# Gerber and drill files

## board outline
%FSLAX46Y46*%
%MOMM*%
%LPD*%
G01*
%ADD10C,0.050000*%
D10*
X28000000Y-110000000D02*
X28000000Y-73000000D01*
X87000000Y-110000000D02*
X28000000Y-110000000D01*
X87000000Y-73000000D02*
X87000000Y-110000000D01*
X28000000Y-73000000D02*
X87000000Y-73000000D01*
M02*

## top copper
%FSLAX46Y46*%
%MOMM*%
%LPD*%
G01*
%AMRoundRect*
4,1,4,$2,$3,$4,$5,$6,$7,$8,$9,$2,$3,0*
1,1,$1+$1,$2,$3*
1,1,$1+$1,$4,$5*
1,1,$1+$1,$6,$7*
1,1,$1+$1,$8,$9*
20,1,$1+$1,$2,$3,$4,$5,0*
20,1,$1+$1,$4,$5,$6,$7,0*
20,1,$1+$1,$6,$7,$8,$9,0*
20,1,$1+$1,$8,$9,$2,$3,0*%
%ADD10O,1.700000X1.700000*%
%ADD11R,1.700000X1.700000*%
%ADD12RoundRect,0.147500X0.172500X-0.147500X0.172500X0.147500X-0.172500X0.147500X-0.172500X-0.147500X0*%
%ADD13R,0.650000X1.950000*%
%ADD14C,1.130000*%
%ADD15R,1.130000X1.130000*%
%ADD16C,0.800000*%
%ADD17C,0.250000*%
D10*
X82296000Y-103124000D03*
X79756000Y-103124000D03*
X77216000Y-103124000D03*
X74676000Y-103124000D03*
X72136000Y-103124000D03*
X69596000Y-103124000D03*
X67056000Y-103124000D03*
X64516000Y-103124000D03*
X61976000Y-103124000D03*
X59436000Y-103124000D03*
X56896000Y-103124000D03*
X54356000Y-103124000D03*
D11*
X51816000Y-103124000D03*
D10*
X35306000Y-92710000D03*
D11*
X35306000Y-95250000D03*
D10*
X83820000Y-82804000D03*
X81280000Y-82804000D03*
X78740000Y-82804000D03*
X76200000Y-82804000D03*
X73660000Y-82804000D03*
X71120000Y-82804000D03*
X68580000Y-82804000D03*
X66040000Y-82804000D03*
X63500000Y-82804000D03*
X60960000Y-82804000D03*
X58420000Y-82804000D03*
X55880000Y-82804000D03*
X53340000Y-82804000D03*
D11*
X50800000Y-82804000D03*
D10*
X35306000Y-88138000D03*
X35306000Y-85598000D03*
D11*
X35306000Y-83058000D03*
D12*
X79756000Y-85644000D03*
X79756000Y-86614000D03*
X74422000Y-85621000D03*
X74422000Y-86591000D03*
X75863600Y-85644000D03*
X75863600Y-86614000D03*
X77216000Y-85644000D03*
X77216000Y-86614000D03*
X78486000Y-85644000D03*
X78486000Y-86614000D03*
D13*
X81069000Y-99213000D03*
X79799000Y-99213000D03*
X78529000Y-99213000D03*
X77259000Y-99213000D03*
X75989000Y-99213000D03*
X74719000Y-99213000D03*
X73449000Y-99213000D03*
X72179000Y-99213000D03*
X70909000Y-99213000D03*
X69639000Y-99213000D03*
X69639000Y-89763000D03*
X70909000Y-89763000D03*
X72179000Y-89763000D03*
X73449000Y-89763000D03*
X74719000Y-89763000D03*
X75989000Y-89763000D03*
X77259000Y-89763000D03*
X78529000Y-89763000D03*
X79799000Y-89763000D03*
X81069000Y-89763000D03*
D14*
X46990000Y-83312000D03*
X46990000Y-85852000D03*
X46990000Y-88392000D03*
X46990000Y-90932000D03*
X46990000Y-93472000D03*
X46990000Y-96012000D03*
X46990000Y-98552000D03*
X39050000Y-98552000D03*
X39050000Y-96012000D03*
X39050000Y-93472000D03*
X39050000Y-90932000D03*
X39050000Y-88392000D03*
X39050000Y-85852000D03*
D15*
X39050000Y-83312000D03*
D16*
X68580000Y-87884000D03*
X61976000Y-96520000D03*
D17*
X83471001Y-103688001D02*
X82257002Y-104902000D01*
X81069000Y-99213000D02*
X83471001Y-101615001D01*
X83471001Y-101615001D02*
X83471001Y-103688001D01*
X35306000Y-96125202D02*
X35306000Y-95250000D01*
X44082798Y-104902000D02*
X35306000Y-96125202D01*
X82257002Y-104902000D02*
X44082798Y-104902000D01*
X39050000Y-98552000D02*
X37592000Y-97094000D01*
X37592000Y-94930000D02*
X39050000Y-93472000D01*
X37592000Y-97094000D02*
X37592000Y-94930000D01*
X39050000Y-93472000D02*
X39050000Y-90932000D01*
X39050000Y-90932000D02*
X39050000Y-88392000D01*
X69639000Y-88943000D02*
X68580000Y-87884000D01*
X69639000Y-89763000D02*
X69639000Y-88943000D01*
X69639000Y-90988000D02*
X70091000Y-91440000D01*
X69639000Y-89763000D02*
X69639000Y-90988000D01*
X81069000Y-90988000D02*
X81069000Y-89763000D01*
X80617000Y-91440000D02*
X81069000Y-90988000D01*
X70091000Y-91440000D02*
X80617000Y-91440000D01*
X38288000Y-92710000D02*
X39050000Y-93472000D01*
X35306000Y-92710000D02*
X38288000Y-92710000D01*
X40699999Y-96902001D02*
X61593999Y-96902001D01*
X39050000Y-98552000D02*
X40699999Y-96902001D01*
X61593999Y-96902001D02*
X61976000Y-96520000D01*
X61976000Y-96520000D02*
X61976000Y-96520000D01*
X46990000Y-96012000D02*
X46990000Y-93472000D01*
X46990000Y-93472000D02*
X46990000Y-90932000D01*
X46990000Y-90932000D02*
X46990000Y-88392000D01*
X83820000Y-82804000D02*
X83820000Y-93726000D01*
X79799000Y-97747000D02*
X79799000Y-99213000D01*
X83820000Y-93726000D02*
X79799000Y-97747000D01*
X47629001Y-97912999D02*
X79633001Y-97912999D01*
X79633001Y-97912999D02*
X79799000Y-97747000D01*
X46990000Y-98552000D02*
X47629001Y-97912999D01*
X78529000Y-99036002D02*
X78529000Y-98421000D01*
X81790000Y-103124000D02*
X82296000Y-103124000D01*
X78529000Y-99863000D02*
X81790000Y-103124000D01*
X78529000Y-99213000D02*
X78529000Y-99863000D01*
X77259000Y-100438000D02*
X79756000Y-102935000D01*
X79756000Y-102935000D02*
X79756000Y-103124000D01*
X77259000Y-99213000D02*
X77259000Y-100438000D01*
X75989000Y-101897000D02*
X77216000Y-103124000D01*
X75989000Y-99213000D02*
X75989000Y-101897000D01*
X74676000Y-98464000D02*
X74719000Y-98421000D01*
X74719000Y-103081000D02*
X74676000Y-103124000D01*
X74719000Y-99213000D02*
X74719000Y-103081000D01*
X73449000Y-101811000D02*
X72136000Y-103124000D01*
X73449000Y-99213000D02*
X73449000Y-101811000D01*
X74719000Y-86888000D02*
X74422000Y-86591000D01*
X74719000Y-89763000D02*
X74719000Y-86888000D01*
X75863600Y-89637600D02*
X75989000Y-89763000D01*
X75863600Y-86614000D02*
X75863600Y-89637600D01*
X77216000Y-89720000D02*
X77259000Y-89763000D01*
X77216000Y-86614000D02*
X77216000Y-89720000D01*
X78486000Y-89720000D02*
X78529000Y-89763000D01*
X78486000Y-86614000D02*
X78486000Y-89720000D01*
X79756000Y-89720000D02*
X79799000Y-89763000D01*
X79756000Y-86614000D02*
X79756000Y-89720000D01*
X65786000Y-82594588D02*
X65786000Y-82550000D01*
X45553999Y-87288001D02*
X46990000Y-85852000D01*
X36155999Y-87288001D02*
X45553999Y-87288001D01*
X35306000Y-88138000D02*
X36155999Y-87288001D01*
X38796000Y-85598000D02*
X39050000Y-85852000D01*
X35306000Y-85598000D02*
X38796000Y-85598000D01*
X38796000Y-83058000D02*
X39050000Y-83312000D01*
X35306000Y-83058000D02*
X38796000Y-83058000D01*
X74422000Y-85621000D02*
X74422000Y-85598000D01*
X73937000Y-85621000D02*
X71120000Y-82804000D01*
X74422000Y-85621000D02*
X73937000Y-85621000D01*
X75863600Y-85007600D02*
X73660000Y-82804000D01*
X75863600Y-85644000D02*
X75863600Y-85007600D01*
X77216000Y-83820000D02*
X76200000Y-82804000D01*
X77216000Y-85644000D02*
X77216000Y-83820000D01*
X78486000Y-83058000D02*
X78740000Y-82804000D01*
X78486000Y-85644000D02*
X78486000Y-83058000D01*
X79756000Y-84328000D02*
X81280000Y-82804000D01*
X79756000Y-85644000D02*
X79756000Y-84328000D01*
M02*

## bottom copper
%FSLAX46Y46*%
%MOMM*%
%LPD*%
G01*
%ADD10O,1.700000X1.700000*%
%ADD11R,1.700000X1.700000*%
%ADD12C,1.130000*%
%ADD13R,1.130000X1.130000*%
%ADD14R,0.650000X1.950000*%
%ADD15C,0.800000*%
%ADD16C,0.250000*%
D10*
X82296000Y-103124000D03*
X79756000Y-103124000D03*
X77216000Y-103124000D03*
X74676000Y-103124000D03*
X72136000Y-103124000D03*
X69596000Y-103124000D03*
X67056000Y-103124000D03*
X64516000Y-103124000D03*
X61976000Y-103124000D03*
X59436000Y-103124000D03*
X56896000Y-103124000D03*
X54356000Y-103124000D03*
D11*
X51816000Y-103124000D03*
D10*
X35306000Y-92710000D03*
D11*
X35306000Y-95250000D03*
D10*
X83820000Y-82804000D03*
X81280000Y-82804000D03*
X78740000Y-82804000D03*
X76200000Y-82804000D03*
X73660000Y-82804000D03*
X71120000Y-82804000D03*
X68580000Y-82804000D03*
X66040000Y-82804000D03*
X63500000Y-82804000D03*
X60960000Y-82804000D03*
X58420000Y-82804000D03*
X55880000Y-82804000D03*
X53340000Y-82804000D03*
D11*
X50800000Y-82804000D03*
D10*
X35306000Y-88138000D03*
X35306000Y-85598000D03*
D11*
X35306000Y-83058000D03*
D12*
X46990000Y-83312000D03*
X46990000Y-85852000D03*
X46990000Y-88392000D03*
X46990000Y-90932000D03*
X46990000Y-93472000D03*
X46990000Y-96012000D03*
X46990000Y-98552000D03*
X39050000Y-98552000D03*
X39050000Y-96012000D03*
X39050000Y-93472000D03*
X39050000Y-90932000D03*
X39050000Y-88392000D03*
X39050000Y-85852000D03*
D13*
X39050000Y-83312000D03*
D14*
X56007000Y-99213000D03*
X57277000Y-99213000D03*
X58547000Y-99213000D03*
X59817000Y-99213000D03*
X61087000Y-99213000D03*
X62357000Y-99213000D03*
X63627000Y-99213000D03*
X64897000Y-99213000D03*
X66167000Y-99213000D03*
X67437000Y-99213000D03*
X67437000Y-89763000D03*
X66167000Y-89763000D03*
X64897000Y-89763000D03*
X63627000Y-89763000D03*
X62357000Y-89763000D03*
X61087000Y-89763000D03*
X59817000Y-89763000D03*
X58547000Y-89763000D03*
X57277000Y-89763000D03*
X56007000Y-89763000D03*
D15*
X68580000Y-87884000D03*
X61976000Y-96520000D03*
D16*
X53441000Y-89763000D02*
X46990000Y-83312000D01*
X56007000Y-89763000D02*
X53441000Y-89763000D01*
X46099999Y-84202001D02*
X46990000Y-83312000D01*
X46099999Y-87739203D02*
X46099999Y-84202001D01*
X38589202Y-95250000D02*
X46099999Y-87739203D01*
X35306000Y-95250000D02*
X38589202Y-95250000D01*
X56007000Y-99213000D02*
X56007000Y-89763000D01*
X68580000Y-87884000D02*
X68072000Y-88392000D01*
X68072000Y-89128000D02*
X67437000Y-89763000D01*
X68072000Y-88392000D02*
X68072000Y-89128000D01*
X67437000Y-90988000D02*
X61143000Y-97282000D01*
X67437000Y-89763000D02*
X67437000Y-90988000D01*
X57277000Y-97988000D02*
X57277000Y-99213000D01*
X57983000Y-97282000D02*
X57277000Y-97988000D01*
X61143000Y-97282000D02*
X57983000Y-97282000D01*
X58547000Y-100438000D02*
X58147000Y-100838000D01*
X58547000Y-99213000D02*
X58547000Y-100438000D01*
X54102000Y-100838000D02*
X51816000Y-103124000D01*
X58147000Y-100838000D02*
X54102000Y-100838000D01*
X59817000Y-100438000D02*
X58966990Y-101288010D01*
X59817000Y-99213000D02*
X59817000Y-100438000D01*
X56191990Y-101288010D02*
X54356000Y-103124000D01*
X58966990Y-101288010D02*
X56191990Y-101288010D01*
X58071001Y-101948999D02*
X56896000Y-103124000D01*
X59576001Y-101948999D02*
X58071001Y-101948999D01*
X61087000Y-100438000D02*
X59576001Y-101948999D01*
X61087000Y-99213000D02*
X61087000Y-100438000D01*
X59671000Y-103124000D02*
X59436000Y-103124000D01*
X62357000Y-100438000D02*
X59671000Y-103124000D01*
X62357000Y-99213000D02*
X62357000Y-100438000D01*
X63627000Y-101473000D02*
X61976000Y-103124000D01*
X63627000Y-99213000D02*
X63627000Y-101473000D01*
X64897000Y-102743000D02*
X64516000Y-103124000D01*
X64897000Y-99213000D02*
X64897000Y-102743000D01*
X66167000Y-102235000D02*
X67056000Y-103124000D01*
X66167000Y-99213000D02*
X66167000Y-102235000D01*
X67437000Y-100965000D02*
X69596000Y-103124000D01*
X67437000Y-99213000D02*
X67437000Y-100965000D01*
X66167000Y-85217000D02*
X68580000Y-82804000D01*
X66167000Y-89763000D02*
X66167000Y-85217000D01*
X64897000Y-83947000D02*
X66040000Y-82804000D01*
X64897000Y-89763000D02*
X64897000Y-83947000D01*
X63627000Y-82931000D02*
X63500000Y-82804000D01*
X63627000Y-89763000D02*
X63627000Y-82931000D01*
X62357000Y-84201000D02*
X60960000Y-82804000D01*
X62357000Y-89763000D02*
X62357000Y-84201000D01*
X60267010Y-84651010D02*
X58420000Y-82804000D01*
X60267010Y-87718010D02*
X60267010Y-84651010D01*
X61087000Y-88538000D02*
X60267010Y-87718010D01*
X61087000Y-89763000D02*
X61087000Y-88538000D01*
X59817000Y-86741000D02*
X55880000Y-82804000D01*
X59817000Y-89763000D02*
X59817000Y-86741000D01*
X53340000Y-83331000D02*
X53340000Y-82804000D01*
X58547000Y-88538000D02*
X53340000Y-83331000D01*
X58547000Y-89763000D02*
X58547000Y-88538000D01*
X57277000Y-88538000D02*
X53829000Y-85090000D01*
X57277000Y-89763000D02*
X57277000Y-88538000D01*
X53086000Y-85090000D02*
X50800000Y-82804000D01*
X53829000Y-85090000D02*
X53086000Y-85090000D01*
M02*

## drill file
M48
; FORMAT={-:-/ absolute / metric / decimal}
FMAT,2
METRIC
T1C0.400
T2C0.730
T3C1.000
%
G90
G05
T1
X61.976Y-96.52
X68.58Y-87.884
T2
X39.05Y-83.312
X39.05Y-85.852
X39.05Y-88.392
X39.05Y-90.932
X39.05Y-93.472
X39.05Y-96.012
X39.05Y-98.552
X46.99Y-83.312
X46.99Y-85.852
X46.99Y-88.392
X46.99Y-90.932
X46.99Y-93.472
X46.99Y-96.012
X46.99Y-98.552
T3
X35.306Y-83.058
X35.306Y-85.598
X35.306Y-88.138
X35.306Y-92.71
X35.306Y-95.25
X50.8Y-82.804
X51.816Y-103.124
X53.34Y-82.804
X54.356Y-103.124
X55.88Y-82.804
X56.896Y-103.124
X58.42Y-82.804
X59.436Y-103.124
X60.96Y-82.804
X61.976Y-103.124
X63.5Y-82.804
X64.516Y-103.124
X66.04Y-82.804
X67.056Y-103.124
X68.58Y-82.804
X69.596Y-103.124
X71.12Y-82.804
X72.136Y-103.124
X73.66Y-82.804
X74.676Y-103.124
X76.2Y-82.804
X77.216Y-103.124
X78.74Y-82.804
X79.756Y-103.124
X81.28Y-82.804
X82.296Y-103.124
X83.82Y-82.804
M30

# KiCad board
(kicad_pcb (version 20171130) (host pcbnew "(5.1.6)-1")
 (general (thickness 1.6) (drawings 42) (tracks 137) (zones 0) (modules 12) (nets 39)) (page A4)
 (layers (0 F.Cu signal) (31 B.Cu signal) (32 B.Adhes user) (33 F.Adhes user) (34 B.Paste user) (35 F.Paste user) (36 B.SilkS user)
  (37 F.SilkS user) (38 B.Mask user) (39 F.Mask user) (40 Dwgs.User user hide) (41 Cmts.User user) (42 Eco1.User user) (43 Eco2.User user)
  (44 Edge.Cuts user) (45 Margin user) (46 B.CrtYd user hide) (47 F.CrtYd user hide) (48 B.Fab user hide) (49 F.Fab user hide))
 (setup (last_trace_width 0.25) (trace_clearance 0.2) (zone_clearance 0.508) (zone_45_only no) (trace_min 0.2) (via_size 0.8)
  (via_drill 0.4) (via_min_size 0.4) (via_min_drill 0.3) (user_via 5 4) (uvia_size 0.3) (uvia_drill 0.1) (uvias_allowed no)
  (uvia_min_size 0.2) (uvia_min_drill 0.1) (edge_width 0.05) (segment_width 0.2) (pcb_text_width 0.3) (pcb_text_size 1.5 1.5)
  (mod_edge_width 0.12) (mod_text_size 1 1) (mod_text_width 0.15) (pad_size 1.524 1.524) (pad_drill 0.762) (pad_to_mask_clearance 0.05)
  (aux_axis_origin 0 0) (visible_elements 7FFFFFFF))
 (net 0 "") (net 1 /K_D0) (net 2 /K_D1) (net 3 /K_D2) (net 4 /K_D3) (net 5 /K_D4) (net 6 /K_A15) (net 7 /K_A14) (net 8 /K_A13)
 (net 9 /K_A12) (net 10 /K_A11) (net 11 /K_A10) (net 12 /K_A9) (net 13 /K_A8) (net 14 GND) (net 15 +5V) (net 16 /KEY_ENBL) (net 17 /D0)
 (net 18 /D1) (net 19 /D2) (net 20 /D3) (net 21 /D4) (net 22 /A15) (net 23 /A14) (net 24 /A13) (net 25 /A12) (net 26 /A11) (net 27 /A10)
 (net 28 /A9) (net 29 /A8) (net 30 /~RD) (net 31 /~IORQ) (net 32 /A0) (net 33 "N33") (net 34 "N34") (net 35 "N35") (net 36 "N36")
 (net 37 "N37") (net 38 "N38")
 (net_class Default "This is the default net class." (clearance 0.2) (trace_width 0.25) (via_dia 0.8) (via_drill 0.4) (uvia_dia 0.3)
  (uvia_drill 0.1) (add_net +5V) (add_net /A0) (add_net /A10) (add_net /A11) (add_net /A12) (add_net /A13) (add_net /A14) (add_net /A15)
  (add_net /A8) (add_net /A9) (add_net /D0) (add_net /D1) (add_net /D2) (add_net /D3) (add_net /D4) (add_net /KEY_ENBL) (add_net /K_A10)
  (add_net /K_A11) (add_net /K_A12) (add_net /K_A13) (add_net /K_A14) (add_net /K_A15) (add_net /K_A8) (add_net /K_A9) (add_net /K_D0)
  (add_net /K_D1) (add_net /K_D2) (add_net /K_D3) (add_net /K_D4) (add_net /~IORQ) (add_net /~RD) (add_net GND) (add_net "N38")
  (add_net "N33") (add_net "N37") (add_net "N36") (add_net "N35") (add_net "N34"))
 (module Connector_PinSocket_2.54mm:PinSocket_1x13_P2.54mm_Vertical (layer B.Cu) (at 51.816 103.124 270)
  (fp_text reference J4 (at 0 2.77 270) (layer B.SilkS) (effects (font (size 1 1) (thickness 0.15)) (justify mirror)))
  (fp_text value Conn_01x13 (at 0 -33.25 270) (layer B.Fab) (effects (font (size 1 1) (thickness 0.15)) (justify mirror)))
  (pad 13 thru_hole oval (at 0 -30.48 270) (size 1.7 1.7) (drill 1) (layers *.Cu *.Mask) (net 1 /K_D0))
  (pad 12 thru_hole oval (at 0 -27.94 270) (size 1.7 1.7) (drill 1) (layers *.Cu *.Mask) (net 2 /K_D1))
  (pad 11 thru_hole oval (at 0 -25.4 270) (size 1.7 1.7) (drill 1) (layers *.Cu *.Mask) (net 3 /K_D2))
  (pad 10 thru_hole oval (at 0 -22.86 270) (size 1.7 1.7) (drill 1) (layers *.Cu *.Mask) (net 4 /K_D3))
  (pad 9 thru_hole oval (at 0 -20.32 270) (size 1.7 1.7) (drill 1) (layers *.Cu *.Mask) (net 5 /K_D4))
  (pad 8 thru_hole oval (at 0 -17.78 270) (size 1.7 1.7) (drill 1) (layers *.Cu *.Mask) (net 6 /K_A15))
  (pad 7 thru_hole oval (at 0 -15.24 270) (size 1.7 1.7) (drill 1) (layers *.Cu *.Mask) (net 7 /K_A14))
  (pad 6 thru_hole oval (at 0 -12.7 270) (size 1.7 1.7) (drill 1) (layers *.Cu *.Mask) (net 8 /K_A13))
  (pad 5 thru_hole oval (at 0 -10.16 270) (size 1.7 1.7) (drill 1) (layers *.Cu *.Mask) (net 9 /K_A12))
  (pad 4 thru_hole oval (at 0 -7.62 270) (size 1.7 1.7) (drill 1) (layers *.Cu *.Mask) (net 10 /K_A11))
  (pad 3 thru_hole oval (at 0 -5.08 270) (size 1.7 1.7) (drill 1) (layers *.Cu *.Mask) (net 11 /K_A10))
  (pad 2 thru_hole oval (at 0 -2.54 270) (size 1.7 1.7) (drill 1) (layers *.Cu *.Mask) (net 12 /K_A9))
  (pad 1 thru_hole rect (at 0 0 270) (size 1.7 1.7) (drill 1) (layers *.Cu *.Mask) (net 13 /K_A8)))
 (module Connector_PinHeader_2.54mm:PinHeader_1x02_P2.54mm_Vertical (layer F.Cu) (at 35.306 95.25 180)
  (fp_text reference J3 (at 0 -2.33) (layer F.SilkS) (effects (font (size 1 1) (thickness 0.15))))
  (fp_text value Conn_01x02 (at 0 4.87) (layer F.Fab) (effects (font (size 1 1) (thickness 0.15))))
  (pad 2 thru_hole oval (at 0 2.54 180) (size 1.7 1.7) (drill 1) (layers *.Cu *.Mask) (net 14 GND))
  (pad 1 thru_hole rect (at 0 0 180) (size 1.7 1.7) (drill 1) (layers *.Cu *.Mask) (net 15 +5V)))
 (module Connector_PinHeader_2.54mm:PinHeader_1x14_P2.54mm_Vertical (layer F.Cu) (at 50.8 82.804 90)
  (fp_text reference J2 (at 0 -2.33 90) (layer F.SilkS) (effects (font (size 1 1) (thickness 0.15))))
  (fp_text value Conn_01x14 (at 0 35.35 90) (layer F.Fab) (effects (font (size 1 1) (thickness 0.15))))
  (pad 14 thru_hole oval (at 0 33.02 90) (size 1.7 1.7) (drill 1) (layers *.Cu *.Mask) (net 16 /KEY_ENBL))
  (pad 13 thru_hole oval (at 0 30.48 90) (size 1.7 1.7) (drill 1) (layers *.Cu *.Mask) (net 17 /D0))
  (pad 12 thru_hole oval (at 0 27.94 90) (size 1.7 1.7) (drill 1) (layers *.Cu *.Mask) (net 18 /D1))
  (pad 11 thru_hole oval (at 0 25.4 90) (size 1.7 1.7) (drill 1) (layers *.Cu *.Mask) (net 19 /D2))
  (pad 10 thru_hole oval (at 0 22.86 90) (size 1.7 1.7) (drill 1) (layers *.Cu *.Mask) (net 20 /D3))
  (pad 9 thru_hole oval (at 0 20.32 90) (size 1.7 1.7) (drill 1) (layers *.Cu *.Mask) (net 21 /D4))
  (pad 8 thru_hole oval (at 0 17.78 90) (size 1.7 1.7) (drill 1) (layers *.Cu *.Mask) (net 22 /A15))
  (pad 7 thru_hole oval (at 0 15.24 90) (size 1.7 1.7) (drill 1) (layers *.Cu *.Mask) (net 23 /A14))
  (pad 6 thru_hole oval (at 0 12.7 90) (size 1.7 1.7) (drill 1) (layers *.Cu *.Mask) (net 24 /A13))
  (pad 5 thru_hole oval (at 0 10.16 90) (size 1.7 1.7) (drill 1) (layers *.Cu *.Mask) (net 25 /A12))
  (pad 4 thru_hole oval (at 0 7.62 90) (size 1.7 1.7) (drill 1) (layers *.Cu *.Mask) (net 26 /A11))
  (pad 3 thru_hole oval (at 0 5.08 90) (size 1.7 1.7) (drill 1) (layers *.Cu *.Mask) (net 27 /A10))
  (pad 2 thru_hole oval (at 0 2.54 90) (size 1.7 1.7) (drill 1) (layers *.Cu *.Mask) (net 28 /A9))
  (pad 1 thru_hole rect (at 0 0 90) (size 1.7 1.7) (drill 1) (layers *.Cu *.Mask) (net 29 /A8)))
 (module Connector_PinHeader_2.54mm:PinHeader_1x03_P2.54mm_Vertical (layer F.Cu) (at 35.306 83.058)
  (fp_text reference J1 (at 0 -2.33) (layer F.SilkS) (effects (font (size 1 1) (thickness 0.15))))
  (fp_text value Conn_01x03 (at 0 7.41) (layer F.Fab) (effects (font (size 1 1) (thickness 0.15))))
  (pad 3 thru_hole oval (at 0 5.08) (size 1.7 1.7) (drill 1) (layers *.Cu *.Mask) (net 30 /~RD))
  (pad 2 thru_hole oval (at 0 2.54) (size 1.7 1.7) (drill 1) (layers *.Cu *.Mask) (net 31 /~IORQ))
  (pad 1 thru_hole rect (at 0 0) (size 1.7 1.7) (drill 1) (layers *.Cu *.Mask) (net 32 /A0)))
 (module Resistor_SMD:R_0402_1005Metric (layer F.Cu) (at 79.756 86.129 90)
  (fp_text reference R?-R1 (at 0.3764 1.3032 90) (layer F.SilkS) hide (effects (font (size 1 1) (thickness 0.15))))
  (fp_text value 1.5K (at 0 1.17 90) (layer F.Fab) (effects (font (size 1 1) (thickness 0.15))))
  (pad 2 smd roundrect (at 0.485 0 90) (size 0.59 0.64) (layers F.Cu F.Paste F.Mask) (roundrect_rratio 0.25) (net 17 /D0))
  (pad 1 smd roundrect (at -0.485 0 90) (size 0.59 0.64) (layers F.Cu F.Paste F.Mask) (roundrect_rratio 0.25) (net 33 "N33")))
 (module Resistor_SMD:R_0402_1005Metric (layer F.Cu) (at 74.422 86.106 90)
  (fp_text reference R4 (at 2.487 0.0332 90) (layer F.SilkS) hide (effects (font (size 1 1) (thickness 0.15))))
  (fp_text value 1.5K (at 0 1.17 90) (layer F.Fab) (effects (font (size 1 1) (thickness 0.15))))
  (pad 2 smd roundrect (at 0.485 0 90) (size 0.59 0.64) (layers F.Cu F.Paste F.Mask) (roundrect_rratio 0.25) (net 21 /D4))
  (pad 1 smd roundrect (at -0.485 0 90) (size 0.59 0.64) (layers F.Cu F.Paste F.Mask) (roundrect_rratio 0.25) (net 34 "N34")))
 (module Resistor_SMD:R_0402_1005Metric (layer F.Cu) (at 75.8636 86.129 90)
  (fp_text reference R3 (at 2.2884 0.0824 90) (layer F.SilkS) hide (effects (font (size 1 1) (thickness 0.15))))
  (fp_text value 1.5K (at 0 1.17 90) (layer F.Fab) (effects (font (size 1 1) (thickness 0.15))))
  (pad 2 smd roundrect (at 0.485 0 90) (size 0.59 0.64) (layers F.Cu F.Paste F.Mask) (roundrect_rratio 0.25) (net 20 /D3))
  (pad 1 smd roundrect (at -0.485 0 90) (size 0.59 0.64) (layers F.Cu F.Paste F.Mask) (roundrect_rratio 0.25) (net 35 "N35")))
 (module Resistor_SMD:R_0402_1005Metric (layer F.Cu) (at 77.216 86.129 90)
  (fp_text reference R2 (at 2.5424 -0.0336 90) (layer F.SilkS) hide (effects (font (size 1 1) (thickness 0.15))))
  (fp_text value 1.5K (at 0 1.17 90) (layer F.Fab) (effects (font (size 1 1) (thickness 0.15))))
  (pad 2 smd roundrect (at 0.485 0 90) (size 0.59 0.64) (layers F.Cu F.Paste F.Mask) (roundrect_rratio 0.25) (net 19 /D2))
  (pad 1 smd roundrect (at -0.485 0 90) (size 0.59 0.64) (layers F.Cu F.Paste F.Mask) (roundrect_rratio 0.25) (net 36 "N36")))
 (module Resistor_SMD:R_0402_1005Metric (layer F.Cu) (at 78.486 86.129 90)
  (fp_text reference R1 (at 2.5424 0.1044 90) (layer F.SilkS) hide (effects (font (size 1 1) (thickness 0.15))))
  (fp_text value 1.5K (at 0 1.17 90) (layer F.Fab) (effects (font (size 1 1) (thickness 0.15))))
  (pad 2 smd roundrect (at 0.485 0 90) (size 0.59 0.64) (layers F.Cu F.Paste F.Mask) (roundrect_rratio 0.25) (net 18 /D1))
  (pad 1 smd roundrect (at -0.485 0 90) (size 0.59 0.64) (layers F.Cu F.Paste F.Mask) (roundrect_rratio 0.25) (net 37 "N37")))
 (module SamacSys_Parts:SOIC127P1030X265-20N (layer F.Cu) (at 75.354 94.488 270)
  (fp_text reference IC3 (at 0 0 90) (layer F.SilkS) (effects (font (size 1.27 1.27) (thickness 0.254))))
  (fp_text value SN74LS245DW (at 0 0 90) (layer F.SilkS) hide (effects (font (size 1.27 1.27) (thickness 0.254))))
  (pad 20 smd rect (at 4.725 -5.715) (size 0.65 1.95) (layers F.Cu F.Paste F.Mask) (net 15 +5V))
  (pad 19 smd rect (at 4.725 -4.445) (size 0.65 1.95) (layers F.Cu F.Paste F.Mask) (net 16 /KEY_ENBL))
  (pad 18 smd rect (at 4.725 -3.175) (size 0.65 1.95) (layers F.Cu F.Paste F.Mask) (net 1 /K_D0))
  (pad 17 smd rect (at 4.725 -1.905) (size 0.65 1.95) (layers F.Cu F.Paste F.Mask) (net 2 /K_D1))
  (pad 16 smd rect (at 4.725 -0.635) (size 0.65 1.95) (layers F.Cu F.Paste F.Mask) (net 3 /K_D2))
  (pad 15 smd rect (at 4.725 0.635) (size 0.65 1.95) (layers F.Cu F.Paste F.Mask) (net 4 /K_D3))
  (pad 14 smd rect (at 4.725 1.905) (size 0.65 1.95) (layers F.Cu F.Paste F.Mask) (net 5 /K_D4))
  (pad 13 smd rect (at 4.725 3.175) (size 0.65 1.95) (layers F.Cu F.Paste F.Mask))
  (pad 12 smd rect (at 4.725 4.445) (size 0.65 1.95) (layers F.Cu F.Paste F.Mask))
  (pad 11 smd rect (at 4.725 5.715) (size 0.65 1.95) (layers F.Cu F.Paste F.Mask))
  (pad 10 smd rect (at -4.725 5.715) (size 0.65 1.95) (layers F.Cu F.Paste F.Mask) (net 14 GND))
  (pad 9 smd rect (at -4.725 4.445) (size 0.65 1.95) (layers F.Cu F.Paste F.Mask))
  (pad 8 smd rect (at -4.725 3.175) (size 0.65 1.95) (layers F.Cu F.Paste F.Mask))
  (pad 7 smd rect (at -4.725 1.905) (size 0.65 1.95) (layers F.Cu F.Paste F.Mask))
  (pad 6 smd rect (at -4.725 0.635) (size 0.65 1.95) (layers F.Cu F.Paste F.Mask) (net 34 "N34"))
  (pad 5 smd rect (at -4.725 -0.635) (size 0.65 1.95) (layers F.Cu F.Paste F.Mask) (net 35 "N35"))
  (pad 4 smd rect (at -4.725 -1.905) (size 0.65 1.95) (layers F.Cu F.Paste F.Mask) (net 36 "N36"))
  (pad 3 smd rect (at -4.725 -3.175) (size 0.65 1.95) (layers F.Cu F.Paste F.Mask) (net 37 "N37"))
  (pad 2 smd rect (at -4.725 -4.445) (size 0.65 1.95) (layers F.Cu F.Paste F.Mask) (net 33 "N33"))
  (pad 1 smd rect (at -4.725 -5.715) (size 0.65 1.95) (layers F.Cu F.Paste F.Mask) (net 14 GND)))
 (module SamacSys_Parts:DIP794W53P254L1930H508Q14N (layer F.Cu) (at 43.02 90.932)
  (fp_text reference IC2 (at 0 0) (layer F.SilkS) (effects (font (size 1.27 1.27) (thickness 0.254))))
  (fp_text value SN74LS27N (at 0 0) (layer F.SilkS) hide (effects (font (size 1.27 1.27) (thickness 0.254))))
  (pad 14 thru_hole circle (at 3.97 -7.62) (size 1.13 1.13) (drill 0.73) (layers *.Cu *.Mask) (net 15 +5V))
  (pad 13 thru_hole circle (at 3.97 -5.08) (size 1.13 1.13) (drill 0.73) (layers *.Cu *.Mask) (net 30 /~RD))
  (pad 12 thru_hole circle (at 3.97 -2.54) (size 1.13 1.13) (drill 0.73) (layers *.Cu *.Mask) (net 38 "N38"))
  (pad 11 thru_hole circle (at 3.97 0) (size 1.13 1.13) (drill 0.73) (layers *.Cu *.Mask) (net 38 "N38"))
  (pad 10 thru_hole circle (at 3.97 2.54) (size 1.13 1.13) (drill 0.73) (layers *.Cu *.Mask) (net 38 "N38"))
  (pad 9 thru_hole circle (at 3.97 5.08) (size 1.13 1.13) (drill 0.73) (layers *.Cu *.Mask) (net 38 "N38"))
  (pad 8 thru_hole circle (at 3.97 7.62) (size 1.13 1.13) (drill 0.73) (layers *.Cu *.Mask) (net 16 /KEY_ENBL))
  (pad 7 thru_hole circle (at -3.97 7.62) (size 1.13 1.13) (drill 0.73) (layers *.Cu *.Mask) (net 14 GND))
  (pad 6 thru_hole circle (at -3.97 5.08) (size 1.13 1.13) (drill 0.73) (layers *.Cu *.Mask))
  (pad 5 thru_hole circle (at -3.97 2.54) (size 1.13 1.13) (drill 0.73) (layers *.Cu *.Mask) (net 14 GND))
  (pad 4 thru_hole circle (at -3.97 0) (size 1.13 1.13) (drill 0.73) (layers *.Cu *.Mask) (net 14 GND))
  (pad 3 thru_hole circle (at -3.97 -2.54) (size 1.13 1.13) (drill 0.73) (layers *.Cu *.Mask) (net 14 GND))
  (pad 2 thru_hole circle (at -3.97 -5.08) (size 1.13 1.13) (drill 0.73) (layers *.Cu *.Mask) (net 31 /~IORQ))
  (pad 1 thru_hole rect (at -3.97 -7.62) (size 1.13 1.13) (drill 0.73) (layers *.Cu *.Mask) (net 32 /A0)))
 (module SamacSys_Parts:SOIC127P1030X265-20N (layer B.Cu) (at 61.722 94.488 270)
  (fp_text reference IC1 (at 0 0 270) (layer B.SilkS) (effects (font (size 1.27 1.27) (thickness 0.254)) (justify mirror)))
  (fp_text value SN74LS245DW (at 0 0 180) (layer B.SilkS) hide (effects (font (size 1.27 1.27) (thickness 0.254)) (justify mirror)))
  (pad 20 smd rect (at 4.725 5.715 180) (size 0.65 1.95) (layers B.Cu B.Paste B.Mask) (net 15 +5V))
  (pad 19 smd rect (at 4.725 4.445 180) (size 0.65 1.95) (layers B.Cu B.Paste B.Mask) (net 14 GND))
  (pad 18 smd rect (at 4.725 3.175 180) (size 0.65 1.95) (layers B.Cu B.Paste B.Mask) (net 13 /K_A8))
  (pad 17 smd rect (at 4.725 1.905 180) (size 0.65 1.95) (layers B.Cu B.Paste B.Mask) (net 12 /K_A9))
  (pad 16 smd rect (at 4.725 0.635 180) (size 0.65 1.95) (layers B.Cu B.Paste B.Mask) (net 11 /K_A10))
  (pad 15 smd rect (at 4.725 -0.635 180) (size 0.65 1.95) (layers B.Cu B.Paste B.Mask) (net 10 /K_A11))
  (pad 14 smd rect (at 4.725 -1.905 180) (size 0.65 1.95) (layers B.Cu B.Paste B.Mask) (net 9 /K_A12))
  (pad 13 smd rect (at 4.725 -3.175 180) (size 0.65 1.95) (layers B.Cu B.Paste B.Mask) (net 8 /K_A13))
  (pad 12 smd rect (at 4.725 -4.445 180) (size 0.65 1.95) (layers B.Cu B.Paste B.Mask) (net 7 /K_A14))
  (pad 11 smd rect (at 4.725 -5.715 180) (size 0.65 1.95) (layers B.Cu B.Paste B.Mask) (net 6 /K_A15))
  (pad 10 smd rect (at -4.725 -5.715 180) (size 0.65 1.95) (layers B.Cu B.Paste B.Mask) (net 14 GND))
  (pad 9 smd rect (at -4.725 -4.445 180) (size 0.65 1.95) (layers B.Cu B.Paste B.Mask) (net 22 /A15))
  (pad 8 smd rect (at -4.725 -3.175 180) (size 0.65 1.95) (layers B.Cu B.Paste B.Mask) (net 23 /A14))
  (pad 7 smd rect (at -4.725 -1.905 180) (size 0.65 1.95) (layers B.Cu B.Paste B.Mask) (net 24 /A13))
  (pad 6 smd rect (at -4.725 -0.635 180) (size 0.65 1.95) (layers B.Cu B.Paste B.Mask) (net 25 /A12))
  (pad 5 smd rect (at -4.725 0.635 180) (size 0.65 1.95) (layers B.Cu B.Paste B.Mask) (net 26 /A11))
  (pad 4 smd rect (at -4.725 1.905 180) (size 0.65 1.95) (layers B.Cu B.Paste B.Mask) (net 27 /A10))
  (pad 3 smd rect (at -4.725 3.175 180) (size 0.65 1.95) (layers B.Cu B.Paste B.Mask) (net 28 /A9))
  (pad 2 smd rect (at -4.725 4.445 180) (size 0.65 1.95) (layers B.Cu B.Paste B.Mask) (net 29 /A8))
  (pad 1 smd rect (at -4.725 5.715 180) (size 0.65 1.95) (layers B.Cu B.Paste B.Mask) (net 15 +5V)))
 (gr_line (start 28 110) (end 28 73) (layer Edge.Cuts) (width 0.05))
 (gr_line (start 87 110) (end 28 110) (layer Edge.Cuts) (width 0.05))
 (gr_line (start 87 73) (end 87 110) (layer Edge.Cuts) (width 0.05))
 (gr_line (start 28 73) (end 87 73) (layer Edge.Cuts) (width 0.05))
 (segment (start 53.441 89.763) (end 46.99 83.312) (width 0.25) (layer B.Cu) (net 15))
 (segment (start 56.007 89.763) (end 53.441 89.763) (width 0.25) (layer B.Cu) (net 15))
 (segment (start 46.099999 84.202001) (end 46.99 83.312) (width 0.25) (layer B.Cu) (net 15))
 (segment (start 46.099999 87.739203) (end 46.099999 84.202001) (width 0.25) (layer B.Cu) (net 15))
 (segment (start 38.589202 95.25) (end 46.099999 87.739203) (width 0.25) (layer B.Cu) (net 15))
 (segment (start 35.306 95.25) (end 38.589202 95.25) (width 0.25) (layer B.Cu) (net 15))
 (segment (start 56.007 99.213) (end 56.007 89.763) (width 0.25) (layer B.Cu) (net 15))
 (segment (start 83.471001 103.688001) (end 82.257002 104.902) (width 0.25) (layer F.Cu) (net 15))
 (segment (start 81.069 99.213) (end 83.471001 101.615001) (width 0.25) (layer F.Cu) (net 15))
 (segment (start 83.471001 101.615001) (end 83.471001 103.688001) (width 0.25) (layer F.Cu) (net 15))
 (segment (start 35.306 96.125202) (end 35.306 95.25) (width 0.25) (layer F.Cu) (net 15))
 (segment (start 44.082798 104.902) (end 35.306 96.125202) (width 0.25) (layer F.Cu) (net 15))
 (segment (start 82.257002 104.902) (end 44.082798 104.902) (width 0.25) (layer F.Cu) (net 15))
 (via (at 68.58 87.884) (size 0.8) (drill 0.4) (layers F.Cu B.Cu) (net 14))
 (segment (start 39.05 98.552) (end 37.592 97.094) (width 0.25) (layer F.Cu) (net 14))
 (segment (start 37.592 94.93) (end 39.05 93.472) (width 0.25) (layer F.Cu) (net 14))
 (segment (start 37.592 97.094) (end 37.592 94.93) (width 0.25) (layer F.Cu) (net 14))
 (segment (start 39.05 93.472) (end 39.05 90.932) (width 0.25) (layer F.Cu) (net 14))
 (segment (start 39.05 90.932) (end 39.05 88.392) (width 0.25) (layer F.Cu) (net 14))
 (segment (start 69.639 88.943) (end 68.58 87.884) (width 0.25) (layer F.Cu) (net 14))
 (segment (start 69.639 89.763) (end 69.639 88.943) (width 0.25) (layer F.Cu) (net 14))
 (segment (start 68.58 87.884) (end 68.072 88.392) (width 0.25) (layer B.Cu) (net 14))
 (segment (start 68.072 89.128) (end 67.437 89.763) (width 0.25) (layer B.Cu) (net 14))
 (segment (start 68.072 88.392) (end 68.072 89.128) (width 0.25) (layer B.Cu) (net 14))
 (segment (start 67.437 90.988) (end 61.143 97.282) (width 0.25) (layer B.Cu) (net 14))
 (segment (start 67.437 89.763) (end 67.437 90.988) (width 0.25) (layer B.Cu) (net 14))
 (segment (start 57.277 97.988) (end 57.277 99.213) (width 0.25) (layer B.Cu) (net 14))
 (segment (start 57.983 97.282) (end 57.277 97.988) (width 0.25) (layer B.Cu) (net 14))
 (segment (start 61.143 97.282) (end 57.983 97.282) (width 0.25) (layer B.Cu) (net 14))
 (segment (start 69.639 90.988) (end 70.091 91.44) (width 0.25) (layer F.Cu) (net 14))
 (segment (start 69.639 89.763) (end 69.639 90.988) (width 0.25) (layer F.Cu) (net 14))
 (segment (start 81.069 90.988) (end 81.069 89.763) (width 0.25) (layer F.Cu) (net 14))
 (segment (start 80.617 91.44) (end 81.069 90.988) (width 0.25) (layer F.Cu) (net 14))
 (segment (start 70.091 91.44) (end 80.617 91.44) (width 0.25) (layer F.Cu) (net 14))
 (segment (start 38.288 92.71) (end 39.05 93.472) (width 0.25) (layer F.Cu) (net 14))
 (segment (start 35.306 92.71) (end 38.288 92.71) (width 0.25) (layer F.Cu) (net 14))
 (segment (start 40.699999 96.902001) (end 61.593999 96.902001) (width 0.25) (layer F.Cu) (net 14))
 (segment (start 39.05 98.552) (end 40.699999 96.902001) (width 0.25) (layer F.Cu) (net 14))
 (segment (start 61.593999 96.902001) (end 61.976 96.52) (width 0.25) (layer F.Cu) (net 14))
 (segment (start 61.976 96.52) (end 61.976 96.52) (width 0.25) (layer F.Cu) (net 14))
 (via (at 61.976 96.52) (size 0.8) (drill 0.4) (layers F.Cu B.Cu) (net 14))
 (segment (start 58.547 100.438) (end 58.147 100.838) (width 0.25) (layer B.Cu) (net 13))
 (segment (start 58.547 99.213) (end 58.547 100.438) (width 0.25) (layer B.Cu) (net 13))
 (segment (start 54.102 100.838) (end 51.816 103.124) (width 0.25) (layer B.Cu) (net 13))
 (segment (start 58.147 100.838) (end 54.102 100.838) (width 0.25) (layer B.Cu) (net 13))
 (segment (start 59.817 100.438) (end 58.96699 101.28801) (width 0.25) (layer B.Cu) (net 12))
 (segment (start 59.817 99.213) (end 59.817 100.438) (width 0.25) (layer B.Cu) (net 12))
 (segment (start 56.19199 101.28801) (end 54.356 103.124) (width 0.25) (layer B.Cu) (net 12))
 (segment (start 58.96699 101.28801) (end 56.19199 101.28801) (width 0.25) (layer B.Cu) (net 12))
 (segment (start 58.071001 101.948999) (end 56.896 103.124) (width 0.25) (layer B.Cu) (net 11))
 (segment (start 59.576001 101.948999) (end 58.071001 101.948999) (width 0.25) (layer B.Cu) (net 11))
 (segment (start 61.087 100.438) (end 59.576001 101.948999) (width 0.25) (layer B.Cu) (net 11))
 (segment (start 61.087 99.213) (end 61.087 100.438) (width 0.25) (layer B.Cu) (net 11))
 (segment (start 59.671 103.124) (end 59.436 103.124) (width 0.25) (layer B.Cu) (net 10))
 (segment (start 62.357 100.438) (end 59.671 103.124) (width 0.25) (layer B.Cu) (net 10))
 (segment (start 62.357 99.213) (end 62.357 100.438) (width 0.25) (layer B.Cu) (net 10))
 (segment (start 63.627 101.473) (end 61.976 103.124) (width 0.25) (layer B.Cu) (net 9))
 (segment (start 63.627 99.213) (end 63.627 101.473) (width 0.25) (layer B.Cu) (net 9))
 (segment (start 64.897 102.743) (end 64.516 103.124) (width 0.25) (layer B.Cu) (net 8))
 (segment (start 64.897 99.213) (end 64.897 102.743) (width 0.25) (layer B.Cu) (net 8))
 (segment (start 66.167 102.235) (end 67.056 103.124) (width 0.25) (layer B.Cu) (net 7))
 (segment (start 66.167 99.213) (end 66.167 102.235) (width 0.25) (layer B.Cu) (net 7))
 (segment (start 67.437 100.965) (end 69.596 103.124) (width 0.25) (layer B.Cu) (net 6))
 (segment (start 67.437 99.213) (end 67.437 100.965) (width 0.25) (layer B.Cu) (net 6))
 (segment (start 46.99 96.012) (end 46.99 93.472) (width 0.25) (layer F.Cu) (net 38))
 (segment (start 46.99 93.472) (end 46.99 90.932) (width 0.25) (layer F.Cu) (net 38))
 (segment (start 46.99 90.932) (end 46.99 88.392) (width 0.25) (layer F.Cu) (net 38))
 (segment (start 83.82 82.804) (end 83.82 93.726) (width 0.25) (layer F.Cu) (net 16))
 (segment (start 79.799 97.747) (end 79.799 99.213) (width 0.25) (layer F.Cu) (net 16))
 (segment (start 83.82 93.726) (end 79.799 97.747) (width 0.25) (layer F.Cu) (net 16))
 (segment (start 47.629001 97.912999) (end 79.633001 97.912999) (width 0.25) (layer F.Cu) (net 16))
 (segment (start 79.633001 97.912999) (end 79.799 97.747) (width 0.25) (layer F.Cu) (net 16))
 (segment (start 46.99 98.552) (end 47.629001 97.912999) (width 0.25) (layer F.Cu) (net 16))
 (segment (start 78.529 99.036002) (end 78.529 98.421) (width 0.25) (layer F.Cu) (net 1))
 (segment (start 81.79 103.124) (end 82.296 103.124) (width 0.25) (layer F.Cu) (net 1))
 (segment (start 78.529 99.863) (end 81.79 103.124) (width 0.25) (layer F.Cu) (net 1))
 (segment (start 78.529 99.213) (end 78.529 99.863) (width 0.25) (layer F.Cu) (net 1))
 (segment (start 77.259 100.438) (end 79.756 102.935) (width 0.25) (layer F.Cu) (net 2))
 (segment (start 79.756 102.935) (end 79.756 103.124) (width 0.25) (layer F.Cu) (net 2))
 (segment (start 77.259 99.213) (end 77.259 100.438) (width 0.25) (layer F.Cu) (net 2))
 (segment (start 75.989 101.897) (end 77.216 103.124) (width 0.25) (layer F.Cu) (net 3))
 (segment (start 75.989 99.213) (end 75.989 101.897) (width 0.25) (layer F.Cu) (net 3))
 (segment (start 74.676 98.464) (end 74.719 98.421) (width 0.25) (layer F.Cu) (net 4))
 (segment (start 74.719 103.081) (end 74.676 103.124) (width 0.25) (layer F.Cu) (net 4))
 (segment (start 74.719 99.213) (end 74.719 103.081) (width 0.25) (layer F.Cu) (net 4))
 (segment (start 73.449 101.811) (end 72.136 103.124) (width 0.25) (layer F.Cu) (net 5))
 (segment (start 73.449 99.213) (end 73.449 101.811) (width 0.25) (layer F.Cu) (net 5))
 (segment (start 74.719 86.888) (end 74.422 86.591) (width 0.25) (layer F.Cu) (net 34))
 (segment (start 74.719 89.763) (end 74.719 86.888) (width 0.25) (layer F.Cu) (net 34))
 (segment (start 75.8636 89.6376) (end 75.989 89.763) (width 0.25) (layer F.Cu) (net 35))
 (segment (start 75.8636 86.614) (end 75.8636 89.6376) (width 0.25) (layer F.Cu) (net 35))
 (segment (start 77.216 89.72) (end 77.259 89.763) (width 0.25) (layer F.Cu) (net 36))
 (segment (start 77.216 86.614) (end 77.216 89.72) (width 0.25) (layer F.Cu) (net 36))
 (segment (start 78.486 89.72) (end 78.529 89.763) (width 0.25) (layer F.Cu) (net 37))
 (segment (start 78.486 86.614) (end 78.486 89.72) (width 0.25) (layer F.Cu) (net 37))
 (segment (start 79.756 89.72) (end 79.799 89.763) (width 0.25) (layer F.Cu) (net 33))
 (segment (start 79.756 86.614) (end 79.756 89.72) (width 0.25) (layer F.Cu) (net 33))
 (segment (start 66.167 85.217) (end 68.58 82.804) (width 0.25) (layer B.Cu) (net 22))
 (segment (start 66.167 89.763) (end 66.167 85.217) (width 0.25) (layer B.Cu) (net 22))
 (segment (start 65.786 82.594588) (end 65.786 82.55) (width 0.25) (layer F.Cu) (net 23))
 (segment (start 64.897 83.947) (end 66.04 82.804) (width 0.25) (layer B.Cu) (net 23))
 (segment (start 64.897 89.763) (end 64.897 83.947) (width 0.25) (layer B.Cu) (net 23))
 (segment (start 63.627 82.931) (end 63.5 82.804) (width 0.25) (layer B.Cu) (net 24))
 (segment (start 63.627 89.763) (end 63.627 82.931) (width 0.25) (layer B.Cu) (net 24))
 (segment (start 62.357 84.201) (end 60.96 82.804) (width 0.25) (layer B.Cu) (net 25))
 (segment (start 62.357 89.763) (end 62.357 84.201) (width 0.25) (layer B.Cu) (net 25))
 (segment (start 60.26701 84.65101) (end 58.42 82.804) (width 0.25) (layer B.Cu) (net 26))
 (segment (start 60.26701 87.71801) (end 60.26701 84.65101) (width 0.25) (layer B.Cu) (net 26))
 (segment (start 61.087 88.538) (end 60.26701 87.71801) (width 0.25) (layer B.Cu) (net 26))
 (segment (start 61.087 89.763) (end 61.087 88.538) (width 0.25) (layer B.Cu) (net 26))
 (segment (start 59.817 86.741) (end 55.88 82.804) (width 0.25) (layer B.Cu) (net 27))
 (segment (start 59.817 89.763) (end 59.817 86.741) (width 0.25) (layer B.Cu) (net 27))
 (segment (start 53.34 83.331) (end 53.34 82.804) (width 0.25) (layer B.Cu) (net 28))
 (segment (start 58.547 88.538) (end 53.34 83.331) (width 0.25) (layer B.Cu) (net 28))
 (segment (start 58.547 89.763) (end 58.547 88.538) (width 0.25) (layer B.Cu) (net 28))
 (segment (start 57.277 88.538) (end 53.829 85.09) (width 0.25) (layer B.Cu) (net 29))
 (segment (start 57.277 89.763) (end 57.277 88.538) (width 0.25) (layer B.Cu) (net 29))
 (segment (start 53.086 85.09) (end 50.8 82.804) (width 0.25) (layer B.Cu) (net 29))
 (segment (start 53.829 85.09) (end 53.086 85.09) (width 0.25) (layer B.Cu) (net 29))
 (segment (start 45.553999 87.288001) (end 46.99 85.852) (width 0.25) (layer F.Cu) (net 30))
 (segment (start 36.155999 87.288001) (end 45.553999 87.288001) (width 0.25) (layer F.Cu) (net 30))
 (segment (start 35.306 88.138) (end 36.155999 87.288001) (width 0.25) (layer F.Cu) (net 30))
 (segment (start 38.796 85.598) (end 39.05 85.852) (width 0.25) (layer F.Cu) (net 31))
 (segment (start 35.306 85.598) (end 38.796 85.598) (width 0.25) (layer F.Cu) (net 31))
 (segment (start 38.796 83.058) (end 39.05 83.312) (width 0.25) (layer F.Cu) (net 32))
 (segment (start 35.306 83.058) (end 38.796 83.058) (width 0.25) (layer F.Cu) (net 32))
 (segment (start 74.422 85.621) (end 74.422 85.598) (width 0.25) (layer F.Cu) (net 21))
 (segment (start 73.937 85.621) (end 71.12 82.804) (width 0.25) (layer F.Cu) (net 21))
 (segment (start 74.422 85.621) (end 73.937 85.621) (width 0.25) (layer F.Cu) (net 21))
 (segment (start 75.8636 85.0076) (end 73.66 82.804) (width 0.25) (layer F.Cu) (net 20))
 (segment (start 75.8636 85.644) (end 75.8636 85.0076) (width 0.25) (layer F.Cu) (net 20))
 (segment (start 77.216 83.82) (end 76.2 82.804) (width 0.25) (layer F.Cu) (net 19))
 (segment (start 77.216 85.644) (end 77.216 83.82) (width 0.25) (layer F.Cu) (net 19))
 (segment (start 78.486 83.058) (end 78.74 82.804) (width 0.25) (layer F.Cu) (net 18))
 (segment (start 78.486 85.644) (end 78.486 83.058) (width 0.25) (layer F.Cu) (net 18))
 (segment (start 79.756 84.328) (end 81.28 82.804) (width 0.25) (layer F.Cu) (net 17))
 (segment (start 79.756 85.644) (end 79.756 84.328) (width 0.25) (layer F.Cu) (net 17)))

